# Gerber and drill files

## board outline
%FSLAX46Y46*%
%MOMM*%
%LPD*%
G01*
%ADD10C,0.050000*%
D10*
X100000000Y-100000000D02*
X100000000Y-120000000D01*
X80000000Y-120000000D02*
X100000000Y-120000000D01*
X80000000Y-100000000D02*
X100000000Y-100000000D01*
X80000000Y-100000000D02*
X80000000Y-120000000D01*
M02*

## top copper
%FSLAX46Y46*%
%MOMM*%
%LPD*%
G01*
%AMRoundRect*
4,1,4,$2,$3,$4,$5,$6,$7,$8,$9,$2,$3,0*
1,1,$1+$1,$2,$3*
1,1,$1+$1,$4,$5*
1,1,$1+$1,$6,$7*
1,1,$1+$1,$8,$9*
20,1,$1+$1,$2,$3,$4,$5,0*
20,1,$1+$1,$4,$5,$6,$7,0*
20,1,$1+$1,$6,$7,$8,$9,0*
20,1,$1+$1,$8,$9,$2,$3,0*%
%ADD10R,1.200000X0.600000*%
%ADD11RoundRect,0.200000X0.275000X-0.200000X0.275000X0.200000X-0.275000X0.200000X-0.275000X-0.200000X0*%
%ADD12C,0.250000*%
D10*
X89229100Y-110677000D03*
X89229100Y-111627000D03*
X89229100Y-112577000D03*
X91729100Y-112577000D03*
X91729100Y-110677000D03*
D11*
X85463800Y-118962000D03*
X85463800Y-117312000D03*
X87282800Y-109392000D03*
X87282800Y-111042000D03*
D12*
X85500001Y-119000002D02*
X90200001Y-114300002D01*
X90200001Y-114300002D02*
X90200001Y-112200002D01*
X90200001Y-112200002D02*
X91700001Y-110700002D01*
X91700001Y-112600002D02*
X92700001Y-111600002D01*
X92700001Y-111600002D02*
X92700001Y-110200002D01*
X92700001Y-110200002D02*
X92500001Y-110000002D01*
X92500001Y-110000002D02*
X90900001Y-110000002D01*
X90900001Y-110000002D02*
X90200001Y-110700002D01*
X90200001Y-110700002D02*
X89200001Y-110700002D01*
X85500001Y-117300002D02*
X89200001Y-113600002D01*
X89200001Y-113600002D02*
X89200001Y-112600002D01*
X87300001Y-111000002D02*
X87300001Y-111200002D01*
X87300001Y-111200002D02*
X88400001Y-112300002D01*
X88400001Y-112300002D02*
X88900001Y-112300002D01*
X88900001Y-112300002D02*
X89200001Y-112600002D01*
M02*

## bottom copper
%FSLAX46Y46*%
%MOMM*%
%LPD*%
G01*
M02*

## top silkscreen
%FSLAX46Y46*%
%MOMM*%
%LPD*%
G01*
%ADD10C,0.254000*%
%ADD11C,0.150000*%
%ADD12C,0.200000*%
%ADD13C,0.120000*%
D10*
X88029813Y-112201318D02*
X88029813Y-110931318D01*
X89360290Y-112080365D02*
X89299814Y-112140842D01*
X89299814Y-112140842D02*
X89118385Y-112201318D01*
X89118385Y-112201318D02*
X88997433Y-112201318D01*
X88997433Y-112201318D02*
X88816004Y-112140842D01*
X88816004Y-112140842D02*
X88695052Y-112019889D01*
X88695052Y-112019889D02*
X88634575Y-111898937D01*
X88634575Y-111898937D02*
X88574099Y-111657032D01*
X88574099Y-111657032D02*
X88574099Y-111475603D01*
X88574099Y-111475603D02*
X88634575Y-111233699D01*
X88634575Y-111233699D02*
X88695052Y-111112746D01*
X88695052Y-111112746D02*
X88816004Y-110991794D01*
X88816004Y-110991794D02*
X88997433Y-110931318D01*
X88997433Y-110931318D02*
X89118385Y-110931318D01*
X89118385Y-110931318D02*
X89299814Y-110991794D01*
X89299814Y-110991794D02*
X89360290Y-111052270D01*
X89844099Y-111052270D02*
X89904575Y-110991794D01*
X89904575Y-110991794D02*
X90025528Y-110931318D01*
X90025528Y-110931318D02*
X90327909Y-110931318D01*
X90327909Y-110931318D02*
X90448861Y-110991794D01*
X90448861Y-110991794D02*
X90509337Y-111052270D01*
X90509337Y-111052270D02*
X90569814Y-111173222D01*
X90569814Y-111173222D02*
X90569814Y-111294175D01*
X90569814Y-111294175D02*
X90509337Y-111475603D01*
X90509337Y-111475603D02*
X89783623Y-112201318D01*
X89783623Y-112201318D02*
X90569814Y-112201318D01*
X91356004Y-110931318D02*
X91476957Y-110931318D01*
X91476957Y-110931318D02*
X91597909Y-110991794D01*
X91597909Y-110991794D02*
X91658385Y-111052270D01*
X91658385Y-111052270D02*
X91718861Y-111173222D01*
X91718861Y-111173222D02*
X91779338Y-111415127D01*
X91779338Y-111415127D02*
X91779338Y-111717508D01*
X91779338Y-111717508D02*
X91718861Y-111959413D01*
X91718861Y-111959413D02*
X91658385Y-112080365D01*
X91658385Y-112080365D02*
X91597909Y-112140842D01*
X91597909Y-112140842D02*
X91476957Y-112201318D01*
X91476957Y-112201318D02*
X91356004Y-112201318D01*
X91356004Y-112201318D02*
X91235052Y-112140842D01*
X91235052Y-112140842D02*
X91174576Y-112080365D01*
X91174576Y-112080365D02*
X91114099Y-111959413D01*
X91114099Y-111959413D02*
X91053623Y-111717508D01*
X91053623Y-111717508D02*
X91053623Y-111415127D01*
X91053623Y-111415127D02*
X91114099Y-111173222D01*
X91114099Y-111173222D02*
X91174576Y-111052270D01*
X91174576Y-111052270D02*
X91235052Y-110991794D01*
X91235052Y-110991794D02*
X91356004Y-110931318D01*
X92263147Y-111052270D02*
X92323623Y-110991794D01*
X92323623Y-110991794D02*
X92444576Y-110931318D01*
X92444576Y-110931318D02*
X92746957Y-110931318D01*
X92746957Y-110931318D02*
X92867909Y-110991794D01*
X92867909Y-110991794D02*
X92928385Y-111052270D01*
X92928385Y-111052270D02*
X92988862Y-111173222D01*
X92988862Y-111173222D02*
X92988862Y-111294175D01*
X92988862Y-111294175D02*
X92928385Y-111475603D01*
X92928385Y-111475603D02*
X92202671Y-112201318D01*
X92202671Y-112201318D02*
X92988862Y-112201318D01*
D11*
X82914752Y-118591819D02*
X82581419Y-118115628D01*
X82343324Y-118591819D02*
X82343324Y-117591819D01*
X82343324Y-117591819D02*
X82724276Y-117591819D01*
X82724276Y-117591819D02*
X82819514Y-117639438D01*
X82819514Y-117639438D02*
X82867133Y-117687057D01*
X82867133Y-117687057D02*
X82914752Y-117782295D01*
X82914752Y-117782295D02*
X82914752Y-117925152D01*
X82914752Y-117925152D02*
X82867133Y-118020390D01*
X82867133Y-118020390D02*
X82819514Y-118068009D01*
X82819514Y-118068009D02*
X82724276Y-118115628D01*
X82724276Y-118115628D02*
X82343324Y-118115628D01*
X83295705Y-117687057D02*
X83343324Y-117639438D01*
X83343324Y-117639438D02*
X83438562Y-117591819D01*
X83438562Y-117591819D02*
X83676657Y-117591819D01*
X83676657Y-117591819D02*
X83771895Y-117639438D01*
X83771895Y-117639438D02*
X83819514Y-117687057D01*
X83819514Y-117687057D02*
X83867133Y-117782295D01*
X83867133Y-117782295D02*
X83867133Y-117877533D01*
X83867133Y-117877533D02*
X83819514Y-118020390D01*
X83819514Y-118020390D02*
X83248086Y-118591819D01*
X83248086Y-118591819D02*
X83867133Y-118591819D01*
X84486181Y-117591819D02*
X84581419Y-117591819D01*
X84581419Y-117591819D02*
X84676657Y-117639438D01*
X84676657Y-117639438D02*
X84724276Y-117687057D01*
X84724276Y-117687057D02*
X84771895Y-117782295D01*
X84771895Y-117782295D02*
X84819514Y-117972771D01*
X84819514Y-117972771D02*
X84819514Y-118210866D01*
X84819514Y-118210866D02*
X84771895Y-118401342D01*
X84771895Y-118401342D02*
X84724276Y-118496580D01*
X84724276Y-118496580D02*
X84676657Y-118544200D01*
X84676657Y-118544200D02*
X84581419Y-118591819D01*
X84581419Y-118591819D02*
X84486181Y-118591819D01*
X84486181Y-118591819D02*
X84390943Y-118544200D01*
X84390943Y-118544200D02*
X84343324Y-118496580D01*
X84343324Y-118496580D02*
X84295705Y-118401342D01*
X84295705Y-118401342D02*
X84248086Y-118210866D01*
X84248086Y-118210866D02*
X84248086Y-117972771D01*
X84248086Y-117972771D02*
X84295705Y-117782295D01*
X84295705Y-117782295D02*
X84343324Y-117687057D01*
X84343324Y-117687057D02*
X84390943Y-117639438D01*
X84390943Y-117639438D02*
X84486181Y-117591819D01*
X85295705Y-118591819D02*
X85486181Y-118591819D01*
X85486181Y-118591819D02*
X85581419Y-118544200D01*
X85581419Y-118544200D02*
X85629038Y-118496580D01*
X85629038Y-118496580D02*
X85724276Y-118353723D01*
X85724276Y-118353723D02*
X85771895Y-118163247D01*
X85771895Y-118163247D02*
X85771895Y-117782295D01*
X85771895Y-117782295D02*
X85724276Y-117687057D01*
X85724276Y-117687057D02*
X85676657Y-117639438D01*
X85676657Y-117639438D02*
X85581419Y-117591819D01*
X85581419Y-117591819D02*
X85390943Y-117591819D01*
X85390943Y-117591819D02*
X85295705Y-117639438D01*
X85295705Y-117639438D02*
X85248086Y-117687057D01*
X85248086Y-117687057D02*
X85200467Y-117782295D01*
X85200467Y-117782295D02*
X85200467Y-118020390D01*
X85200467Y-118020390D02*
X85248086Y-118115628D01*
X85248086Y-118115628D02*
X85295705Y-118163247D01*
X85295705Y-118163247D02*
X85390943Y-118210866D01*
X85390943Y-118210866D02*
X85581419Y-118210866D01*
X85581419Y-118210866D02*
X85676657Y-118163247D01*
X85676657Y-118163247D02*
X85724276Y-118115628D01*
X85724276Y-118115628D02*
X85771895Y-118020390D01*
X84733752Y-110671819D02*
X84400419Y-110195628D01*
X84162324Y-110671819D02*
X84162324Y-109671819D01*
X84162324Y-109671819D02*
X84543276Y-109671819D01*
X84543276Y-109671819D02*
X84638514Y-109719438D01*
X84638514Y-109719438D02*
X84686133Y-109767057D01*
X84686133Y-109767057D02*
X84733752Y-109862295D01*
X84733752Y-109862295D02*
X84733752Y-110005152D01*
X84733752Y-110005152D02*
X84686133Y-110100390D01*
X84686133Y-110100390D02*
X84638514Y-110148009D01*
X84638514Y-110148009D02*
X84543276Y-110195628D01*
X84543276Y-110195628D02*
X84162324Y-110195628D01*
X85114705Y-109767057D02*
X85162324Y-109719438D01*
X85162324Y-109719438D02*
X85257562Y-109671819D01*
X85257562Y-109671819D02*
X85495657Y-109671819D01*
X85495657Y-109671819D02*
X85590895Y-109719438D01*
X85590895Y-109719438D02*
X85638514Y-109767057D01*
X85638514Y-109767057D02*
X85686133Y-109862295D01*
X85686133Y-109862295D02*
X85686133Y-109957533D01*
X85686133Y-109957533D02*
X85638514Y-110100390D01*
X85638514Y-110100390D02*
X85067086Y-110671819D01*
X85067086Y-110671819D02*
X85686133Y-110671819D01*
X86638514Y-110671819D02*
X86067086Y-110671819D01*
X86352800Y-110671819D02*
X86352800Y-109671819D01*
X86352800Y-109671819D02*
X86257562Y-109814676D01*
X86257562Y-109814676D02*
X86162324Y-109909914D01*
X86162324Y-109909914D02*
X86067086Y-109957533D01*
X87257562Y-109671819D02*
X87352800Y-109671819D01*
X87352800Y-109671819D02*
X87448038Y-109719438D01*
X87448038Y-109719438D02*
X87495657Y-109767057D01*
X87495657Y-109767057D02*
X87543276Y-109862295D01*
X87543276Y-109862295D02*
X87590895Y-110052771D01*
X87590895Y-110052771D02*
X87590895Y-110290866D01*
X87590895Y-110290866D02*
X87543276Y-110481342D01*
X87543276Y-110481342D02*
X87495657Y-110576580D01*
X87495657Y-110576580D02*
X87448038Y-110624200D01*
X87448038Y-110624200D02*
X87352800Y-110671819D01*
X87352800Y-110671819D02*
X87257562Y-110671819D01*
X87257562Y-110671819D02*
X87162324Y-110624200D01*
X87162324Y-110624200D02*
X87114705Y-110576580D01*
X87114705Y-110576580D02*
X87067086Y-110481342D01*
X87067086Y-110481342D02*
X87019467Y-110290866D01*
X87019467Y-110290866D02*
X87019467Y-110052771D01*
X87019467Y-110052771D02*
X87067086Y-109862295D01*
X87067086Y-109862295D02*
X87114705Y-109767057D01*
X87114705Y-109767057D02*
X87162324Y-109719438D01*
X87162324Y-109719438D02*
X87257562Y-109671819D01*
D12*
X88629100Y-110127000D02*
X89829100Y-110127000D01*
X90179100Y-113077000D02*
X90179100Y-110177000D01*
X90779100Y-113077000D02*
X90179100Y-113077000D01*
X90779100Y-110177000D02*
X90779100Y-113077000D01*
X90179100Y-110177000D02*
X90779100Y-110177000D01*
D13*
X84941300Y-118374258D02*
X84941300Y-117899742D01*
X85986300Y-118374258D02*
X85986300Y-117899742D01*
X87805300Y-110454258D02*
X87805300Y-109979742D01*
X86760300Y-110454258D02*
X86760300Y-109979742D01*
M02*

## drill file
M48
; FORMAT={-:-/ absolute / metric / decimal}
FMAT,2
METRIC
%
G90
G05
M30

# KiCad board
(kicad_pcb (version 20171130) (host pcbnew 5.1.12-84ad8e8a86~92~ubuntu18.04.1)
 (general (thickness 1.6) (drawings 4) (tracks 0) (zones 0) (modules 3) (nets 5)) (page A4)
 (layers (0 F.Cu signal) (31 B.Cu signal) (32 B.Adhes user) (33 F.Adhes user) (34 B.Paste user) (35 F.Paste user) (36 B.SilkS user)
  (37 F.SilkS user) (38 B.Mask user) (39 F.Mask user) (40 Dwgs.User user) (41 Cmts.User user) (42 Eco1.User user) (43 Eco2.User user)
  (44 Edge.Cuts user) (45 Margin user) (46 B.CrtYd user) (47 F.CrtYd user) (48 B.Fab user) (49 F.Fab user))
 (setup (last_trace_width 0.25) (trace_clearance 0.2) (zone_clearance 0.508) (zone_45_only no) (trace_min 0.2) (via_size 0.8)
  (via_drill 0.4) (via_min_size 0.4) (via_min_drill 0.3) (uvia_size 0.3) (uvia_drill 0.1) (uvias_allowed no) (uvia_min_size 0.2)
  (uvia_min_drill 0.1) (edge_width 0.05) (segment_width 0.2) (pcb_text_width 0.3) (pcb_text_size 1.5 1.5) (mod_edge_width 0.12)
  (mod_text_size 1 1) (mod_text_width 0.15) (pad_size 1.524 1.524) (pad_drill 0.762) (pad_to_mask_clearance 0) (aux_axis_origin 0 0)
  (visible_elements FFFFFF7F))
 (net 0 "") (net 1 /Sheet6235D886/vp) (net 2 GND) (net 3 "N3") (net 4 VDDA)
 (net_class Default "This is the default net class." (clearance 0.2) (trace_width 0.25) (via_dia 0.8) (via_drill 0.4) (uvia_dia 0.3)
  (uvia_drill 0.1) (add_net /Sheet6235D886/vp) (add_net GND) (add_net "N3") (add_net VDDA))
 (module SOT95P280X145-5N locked (layer F.Cu) (at 90.479100 111.627000)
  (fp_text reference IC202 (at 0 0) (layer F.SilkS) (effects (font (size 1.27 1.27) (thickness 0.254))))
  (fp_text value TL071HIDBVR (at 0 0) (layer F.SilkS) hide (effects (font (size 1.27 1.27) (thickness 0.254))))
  (fp_line (start -1.85 -1.5) (end -0.65 -1.5) (layer F.SilkS) (width 0.2))
  (fp_line (start -0.3 1.45) (end -0.3 -1.45) (layer F.SilkS) (width 0.2))
  (fp_line (start 0.3 1.45) (end -0.3 1.45) (layer F.SilkS) (width 0.2))
  (fp_line (start 0.3 -1.45) (end 0.3 1.45) (layer F.SilkS) (width 0.2))
  (fp_line (start -0.3 -1.45) (end 0.3 -1.45) (layer F.SilkS) (width 0.2))
  (pad 1 smd rect (at -1.25 -0.95 90.000000) (size 0.6 1.2) (layers F.Cu F.Mask F.Paste) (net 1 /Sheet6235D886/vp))
  (pad 2 smd rect (at -1.25 0 90.000000) (size 0.6 1.2) (layers F.Cu F.Mask F.Paste) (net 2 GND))
  (pad 3 smd rect (at -1.25 0.95 90.000000) (size 0.6 1.2) (layers F.Cu F.Mask F.Paste) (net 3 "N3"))
  (pad 4 smd rect (at 1.25 0.95 90.000000) (size 0.6 1.2) (layers F.Cu F.Mask F.Paste) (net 1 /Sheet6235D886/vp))
  (pad 5 smd rect (at 1.25 -0.95 90.000000) (size 0.6 1.2) (layers F.Cu F.Mask F.Paste) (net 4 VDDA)))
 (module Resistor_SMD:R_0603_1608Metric (layer F.Cu) (at 85.463800 118.137000 90.000000)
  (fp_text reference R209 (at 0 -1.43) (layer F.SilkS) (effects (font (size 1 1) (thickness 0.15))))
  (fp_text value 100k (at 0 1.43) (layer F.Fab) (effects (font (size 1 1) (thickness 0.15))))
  (fp_line (start -0.237258 -0.5225) (end 0.237258 -0.5225) (layer F.SilkS) (width 0.12))
  (fp_line (start -0.237258 0.5225) (end 0.237258 0.5225) (layer F.SilkS) (width 0.12))
  (pad 1 smd roundrect (at -0.825 0 90.000000) (size 0.8 0.95) (layers F.Cu F.Mask F.Paste) (roundrect_rratio 0.25) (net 4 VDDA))
  (pad 2 smd roundrect (at 0.825 0 90.000000) (size 0.8 0.95) (layers F.Cu F.Mask F.Paste) (roundrect_rratio 0.25) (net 3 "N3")))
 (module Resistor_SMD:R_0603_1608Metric (layer F.Cu) (at 87.282800 110.217000 90.000000)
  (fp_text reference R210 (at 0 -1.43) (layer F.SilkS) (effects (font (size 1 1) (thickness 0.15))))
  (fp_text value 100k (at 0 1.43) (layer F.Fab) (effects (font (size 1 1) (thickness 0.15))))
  (fp_line (start -0.237258 0.5225) (end 0.237258 0.5225) (layer F.SilkS) (width 0.12))
  (fp_line (start -0.237258 -0.5225) (end 0.237258 -0.5225) (layer F.SilkS) (width 0.12))
  (pad 2 smd roundrect (at 0.825 0 90.000000) (size 0.8 0.95) (layers F.Cu F.Mask F.Paste) (roundrect_rratio 0.25) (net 2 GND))
  (pad 1 smd roundrect (at -0.825 0 90.000000) (size 0.8 0.95) (layers F.Cu F.Mask F.Paste) (roundrect_rratio 0.25) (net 3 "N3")))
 (gr_line (start 100 100) (end 100 120) (layer Edge.Cuts) (width 0.05))
 (gr_line (start 80 120) (end 100 120) (layer Edge.Cuts) (width 0.05))
 (gr_line (start 80 100) (end 100 100) (layer Edge.Cuts) (width 0.05))
 (gr_line (start 80 100) (end 80 120) (layer Edge.Cuts) (width 0.05))
 (segment (start 85.500001 119.000002) (end 90.200001 114.300002) (width 0.250000) (layer F.Cu) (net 4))
 (segment (start 90.200001 114.300002) (end 90.200001 112.200002) (width 0.250000) (layer F.Cu) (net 4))
 (segment (start 90.200001 112.200002) (end 91.700001 110.700002) (width 0.250000) (layer F.Cu) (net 4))
 (segment (start 91.700001 112.600002) (end 92.700001 111.600002) (width 0.250000) (layer F.Cu) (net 1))
 (segment (start 92.700001 111.600002) (end 92.700001 110.200002) (width 0.250000) (layer F.Cu) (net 1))
 (segment (start 92.700001 110.200002) (end 92.500001 110.000002) (width 0.250000) (layer F.Cu) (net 1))
 (segment (start 92.500001 110.000002) (end 90.900001 110.000002) (width 0.250000) (layer F.Cu) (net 1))
 (segment (start 90.900001 110.000002) (end 90.200001 110.700002) (width 0.250000) (layer F.Cu) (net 1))
 (segment (start 90.200001 110.700002) (end 89.200001 110.700002) (width 0.250000) (layer F.Cu) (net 1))
 (segment (start 85.500001 117.300002) (end 89.200001 113.600002) (width 0.250000) (layer F.Cu) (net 3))
 (segment (start 89.200001 113.600002) (end 89.200001 112.600002) (width 0.250000) (layer F.Cu) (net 3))
 (segment (start 87.300001 111.000002) (end 87.300001 111.200002) (width 0.250000) (layer F.Cu) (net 3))
 (segment (start 87.300001 111.200002) (end 88.400001 112.300002) (width 0.250000) (layer F.Cu) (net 3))
 (segment (start 88.400001 112.300002) (end 88.900001 112.300002) (width 0.250000) (layer F.Cu) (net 3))
 (segment (start 88.900001 112.300002) (end 89.200001 112.600002) (width 0.250000) (layer F.Cu) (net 3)))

